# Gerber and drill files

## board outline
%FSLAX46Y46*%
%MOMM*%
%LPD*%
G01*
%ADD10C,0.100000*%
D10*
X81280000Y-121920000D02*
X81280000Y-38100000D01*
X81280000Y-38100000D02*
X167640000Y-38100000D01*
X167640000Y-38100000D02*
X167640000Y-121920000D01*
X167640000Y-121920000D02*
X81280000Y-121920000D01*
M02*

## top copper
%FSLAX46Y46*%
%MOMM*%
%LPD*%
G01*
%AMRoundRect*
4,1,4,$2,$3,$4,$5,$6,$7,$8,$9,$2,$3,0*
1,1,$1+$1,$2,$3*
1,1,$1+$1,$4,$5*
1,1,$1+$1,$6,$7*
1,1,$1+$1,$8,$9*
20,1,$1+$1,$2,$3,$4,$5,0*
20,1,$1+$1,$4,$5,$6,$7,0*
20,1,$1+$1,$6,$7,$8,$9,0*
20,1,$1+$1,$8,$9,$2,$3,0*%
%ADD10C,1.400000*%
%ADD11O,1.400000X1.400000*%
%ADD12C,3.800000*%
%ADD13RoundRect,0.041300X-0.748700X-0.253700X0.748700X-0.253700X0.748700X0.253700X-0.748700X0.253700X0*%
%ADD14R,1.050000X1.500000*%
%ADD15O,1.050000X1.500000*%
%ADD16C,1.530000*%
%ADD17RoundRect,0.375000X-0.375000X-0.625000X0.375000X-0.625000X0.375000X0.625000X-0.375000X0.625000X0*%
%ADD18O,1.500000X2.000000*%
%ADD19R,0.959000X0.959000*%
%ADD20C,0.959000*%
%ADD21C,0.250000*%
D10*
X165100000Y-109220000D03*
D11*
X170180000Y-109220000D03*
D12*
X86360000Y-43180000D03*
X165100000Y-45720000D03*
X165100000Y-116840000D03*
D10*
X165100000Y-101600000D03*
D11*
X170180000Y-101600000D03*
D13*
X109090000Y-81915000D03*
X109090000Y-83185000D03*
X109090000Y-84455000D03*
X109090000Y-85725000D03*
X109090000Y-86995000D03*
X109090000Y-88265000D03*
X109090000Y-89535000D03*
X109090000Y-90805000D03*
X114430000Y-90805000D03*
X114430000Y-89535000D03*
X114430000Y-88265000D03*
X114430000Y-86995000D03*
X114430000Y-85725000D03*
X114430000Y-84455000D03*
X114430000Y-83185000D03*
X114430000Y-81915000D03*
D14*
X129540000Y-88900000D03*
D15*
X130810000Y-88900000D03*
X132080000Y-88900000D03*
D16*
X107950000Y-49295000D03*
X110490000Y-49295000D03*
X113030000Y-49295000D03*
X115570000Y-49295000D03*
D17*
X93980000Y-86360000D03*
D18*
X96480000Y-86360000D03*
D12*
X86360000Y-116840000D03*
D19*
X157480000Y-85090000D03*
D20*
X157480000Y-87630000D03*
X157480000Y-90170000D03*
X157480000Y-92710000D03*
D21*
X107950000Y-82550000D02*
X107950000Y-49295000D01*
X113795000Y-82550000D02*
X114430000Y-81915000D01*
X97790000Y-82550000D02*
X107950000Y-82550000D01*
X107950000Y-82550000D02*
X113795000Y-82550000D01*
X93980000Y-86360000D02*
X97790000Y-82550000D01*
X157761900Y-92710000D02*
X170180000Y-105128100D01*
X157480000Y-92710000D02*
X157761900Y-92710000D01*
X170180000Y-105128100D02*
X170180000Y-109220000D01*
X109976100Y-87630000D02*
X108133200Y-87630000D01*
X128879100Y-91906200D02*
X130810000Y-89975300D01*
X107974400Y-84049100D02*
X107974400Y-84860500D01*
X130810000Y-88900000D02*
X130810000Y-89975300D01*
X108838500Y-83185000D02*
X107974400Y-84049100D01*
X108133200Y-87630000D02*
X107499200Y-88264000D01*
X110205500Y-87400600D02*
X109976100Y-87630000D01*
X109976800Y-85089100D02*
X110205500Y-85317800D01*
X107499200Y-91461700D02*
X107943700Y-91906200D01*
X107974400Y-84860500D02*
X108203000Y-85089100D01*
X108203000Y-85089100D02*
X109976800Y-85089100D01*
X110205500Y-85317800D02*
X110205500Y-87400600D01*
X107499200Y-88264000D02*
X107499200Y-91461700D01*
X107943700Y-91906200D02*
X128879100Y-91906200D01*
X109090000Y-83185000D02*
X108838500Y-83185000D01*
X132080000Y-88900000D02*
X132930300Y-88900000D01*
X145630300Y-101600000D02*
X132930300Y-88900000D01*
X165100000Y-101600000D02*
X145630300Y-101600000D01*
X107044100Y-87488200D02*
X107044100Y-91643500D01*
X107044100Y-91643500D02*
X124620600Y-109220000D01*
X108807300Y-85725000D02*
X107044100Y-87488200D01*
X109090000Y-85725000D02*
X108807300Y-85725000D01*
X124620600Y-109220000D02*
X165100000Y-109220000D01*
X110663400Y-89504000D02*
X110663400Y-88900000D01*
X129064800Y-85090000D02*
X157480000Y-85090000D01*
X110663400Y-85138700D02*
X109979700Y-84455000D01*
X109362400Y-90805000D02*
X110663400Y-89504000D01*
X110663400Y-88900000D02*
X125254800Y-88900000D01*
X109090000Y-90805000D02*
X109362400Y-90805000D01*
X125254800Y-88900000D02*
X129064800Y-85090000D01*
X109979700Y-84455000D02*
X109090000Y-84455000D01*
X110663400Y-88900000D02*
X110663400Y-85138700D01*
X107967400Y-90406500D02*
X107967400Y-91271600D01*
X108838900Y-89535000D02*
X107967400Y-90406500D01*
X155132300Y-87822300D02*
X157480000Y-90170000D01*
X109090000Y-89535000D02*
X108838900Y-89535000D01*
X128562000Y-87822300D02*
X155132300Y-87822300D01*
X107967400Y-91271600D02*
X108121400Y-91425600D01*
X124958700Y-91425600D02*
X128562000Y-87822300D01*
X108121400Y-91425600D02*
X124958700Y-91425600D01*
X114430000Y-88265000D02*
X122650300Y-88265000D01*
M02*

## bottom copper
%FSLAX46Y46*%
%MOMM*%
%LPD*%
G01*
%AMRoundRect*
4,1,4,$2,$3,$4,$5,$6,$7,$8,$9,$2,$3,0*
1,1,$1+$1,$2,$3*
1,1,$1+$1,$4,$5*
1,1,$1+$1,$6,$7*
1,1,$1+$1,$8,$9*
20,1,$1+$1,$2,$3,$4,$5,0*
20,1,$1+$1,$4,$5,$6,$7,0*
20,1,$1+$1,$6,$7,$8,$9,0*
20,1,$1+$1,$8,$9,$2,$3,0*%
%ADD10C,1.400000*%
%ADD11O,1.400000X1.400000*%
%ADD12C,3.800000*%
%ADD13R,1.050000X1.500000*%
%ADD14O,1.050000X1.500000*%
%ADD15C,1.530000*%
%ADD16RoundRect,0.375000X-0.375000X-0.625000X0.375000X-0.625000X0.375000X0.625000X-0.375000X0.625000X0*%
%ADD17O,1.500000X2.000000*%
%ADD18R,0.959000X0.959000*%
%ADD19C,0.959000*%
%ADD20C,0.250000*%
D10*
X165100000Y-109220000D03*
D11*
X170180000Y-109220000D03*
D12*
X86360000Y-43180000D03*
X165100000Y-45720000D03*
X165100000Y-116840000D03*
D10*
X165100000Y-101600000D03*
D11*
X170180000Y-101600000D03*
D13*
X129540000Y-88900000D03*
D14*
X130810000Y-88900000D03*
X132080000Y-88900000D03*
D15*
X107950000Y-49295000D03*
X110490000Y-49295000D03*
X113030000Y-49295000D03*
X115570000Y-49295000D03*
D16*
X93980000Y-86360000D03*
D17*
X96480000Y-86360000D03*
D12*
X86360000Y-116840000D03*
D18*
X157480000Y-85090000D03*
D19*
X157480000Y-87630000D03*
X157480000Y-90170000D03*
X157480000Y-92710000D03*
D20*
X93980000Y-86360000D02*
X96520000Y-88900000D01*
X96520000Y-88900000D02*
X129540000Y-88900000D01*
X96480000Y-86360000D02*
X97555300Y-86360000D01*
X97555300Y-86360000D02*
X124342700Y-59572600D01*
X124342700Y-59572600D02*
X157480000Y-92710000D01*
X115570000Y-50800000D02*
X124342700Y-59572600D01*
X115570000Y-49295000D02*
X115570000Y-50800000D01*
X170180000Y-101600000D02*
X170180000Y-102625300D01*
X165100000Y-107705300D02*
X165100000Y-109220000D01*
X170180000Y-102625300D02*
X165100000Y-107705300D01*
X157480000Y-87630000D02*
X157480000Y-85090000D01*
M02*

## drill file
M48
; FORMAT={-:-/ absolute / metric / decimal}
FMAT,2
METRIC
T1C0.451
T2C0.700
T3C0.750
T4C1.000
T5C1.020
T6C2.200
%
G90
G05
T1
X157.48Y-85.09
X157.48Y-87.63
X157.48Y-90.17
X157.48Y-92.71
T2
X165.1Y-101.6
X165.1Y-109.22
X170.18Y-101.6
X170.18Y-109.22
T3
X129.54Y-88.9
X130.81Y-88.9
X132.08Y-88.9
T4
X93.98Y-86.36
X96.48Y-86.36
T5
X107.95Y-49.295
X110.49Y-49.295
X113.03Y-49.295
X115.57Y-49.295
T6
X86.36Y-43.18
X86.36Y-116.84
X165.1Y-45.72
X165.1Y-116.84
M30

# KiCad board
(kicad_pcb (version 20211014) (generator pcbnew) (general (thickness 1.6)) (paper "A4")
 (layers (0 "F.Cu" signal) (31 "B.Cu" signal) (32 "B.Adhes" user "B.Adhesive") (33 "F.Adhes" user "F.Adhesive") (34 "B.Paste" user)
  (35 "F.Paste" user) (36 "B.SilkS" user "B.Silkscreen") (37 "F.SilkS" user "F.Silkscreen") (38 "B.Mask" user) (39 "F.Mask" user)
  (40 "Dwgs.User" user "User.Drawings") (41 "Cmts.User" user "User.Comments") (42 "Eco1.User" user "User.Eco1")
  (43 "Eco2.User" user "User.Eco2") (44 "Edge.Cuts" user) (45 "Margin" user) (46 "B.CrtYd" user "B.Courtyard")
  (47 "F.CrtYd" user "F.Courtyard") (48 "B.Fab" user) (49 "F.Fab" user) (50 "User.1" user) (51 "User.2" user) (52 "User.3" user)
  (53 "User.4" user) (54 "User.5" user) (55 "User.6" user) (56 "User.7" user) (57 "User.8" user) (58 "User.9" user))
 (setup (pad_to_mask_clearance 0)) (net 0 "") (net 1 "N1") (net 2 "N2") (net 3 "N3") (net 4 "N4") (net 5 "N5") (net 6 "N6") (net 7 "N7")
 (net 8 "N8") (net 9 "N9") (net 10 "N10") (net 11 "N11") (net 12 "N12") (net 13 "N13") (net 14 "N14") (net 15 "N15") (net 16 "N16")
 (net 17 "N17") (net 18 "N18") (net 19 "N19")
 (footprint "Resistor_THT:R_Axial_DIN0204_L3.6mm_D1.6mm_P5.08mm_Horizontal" (layer "F.Cu") (at 165.1 109.22)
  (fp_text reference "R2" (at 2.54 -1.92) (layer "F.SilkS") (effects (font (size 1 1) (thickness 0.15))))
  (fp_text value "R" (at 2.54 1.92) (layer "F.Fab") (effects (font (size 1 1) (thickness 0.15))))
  (pad "1" thru_hole circle (at 0 0) (size 1.4 1.4) (drill 0.7) (layers *.Cu *.Mask) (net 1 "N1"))
  (pad "2" thru_hole oval (at 5.08 0) (size 1.4 1.4) (drill 0.7) (layers *.Cu *.Mask) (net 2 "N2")))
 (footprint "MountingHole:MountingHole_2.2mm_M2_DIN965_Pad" (layer "F.Cu") (at 86.36 43.18)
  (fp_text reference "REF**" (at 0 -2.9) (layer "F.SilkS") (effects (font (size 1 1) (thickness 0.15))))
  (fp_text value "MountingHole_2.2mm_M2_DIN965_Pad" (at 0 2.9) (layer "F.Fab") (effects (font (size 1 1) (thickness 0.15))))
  (pad "1" thru_hole circle (at 0 0) (size 3.8 3.8) (drill 2.2) (layers *.Cu *.Mask)))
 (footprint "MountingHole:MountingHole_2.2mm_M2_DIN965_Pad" (layer "F.Cu") (at 165.1 45.72)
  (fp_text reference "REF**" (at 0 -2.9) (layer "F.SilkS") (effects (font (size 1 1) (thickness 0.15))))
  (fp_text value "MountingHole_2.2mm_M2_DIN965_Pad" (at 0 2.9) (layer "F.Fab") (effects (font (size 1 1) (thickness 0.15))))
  (pad "1" thru_hole circle (at 0 0) (size 3.8 3.8) (drill 2.2) (layers *.Cu *.Mask)))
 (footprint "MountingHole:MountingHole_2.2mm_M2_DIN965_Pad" (layer "F.Cu") (at 165.1 116.84)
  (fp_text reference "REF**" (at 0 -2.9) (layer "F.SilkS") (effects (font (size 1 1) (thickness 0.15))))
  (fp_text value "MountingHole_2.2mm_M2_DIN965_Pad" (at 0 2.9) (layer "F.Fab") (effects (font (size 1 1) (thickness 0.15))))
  (pad "1" thru_hole circle (at 0 0) (size 3.8 3.8) (drill 2.2) (layers *.Cu *.Mask)))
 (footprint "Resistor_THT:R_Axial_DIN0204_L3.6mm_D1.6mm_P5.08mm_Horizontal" (layer "F.Cu") (at 165.1 101.6)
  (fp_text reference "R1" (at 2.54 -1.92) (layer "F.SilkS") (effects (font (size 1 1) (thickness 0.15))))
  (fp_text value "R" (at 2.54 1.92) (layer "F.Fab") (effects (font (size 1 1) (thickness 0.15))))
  (pad "1" thru_hole circle (at 0 0) (size 1.4 1.4) (drill 0.7) (layers *.Cu *.Mask) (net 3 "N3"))
  (pad "2" thru_hole oval (at 5.08 0) (size 1.4 1.4) (drill 0.7) (layers *.Cu *.Mask) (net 1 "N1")))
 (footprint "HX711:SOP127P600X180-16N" (layer "F.Cu") (at 111.76 86.36)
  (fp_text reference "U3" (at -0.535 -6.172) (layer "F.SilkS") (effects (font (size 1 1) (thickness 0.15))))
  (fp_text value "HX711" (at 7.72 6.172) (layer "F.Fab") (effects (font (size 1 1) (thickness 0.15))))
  (pad "1" smd roundrect locked (at -2.67 -4.445) (size 1.58 0.59) (layers "F.Cu" "F.Paste" "F.Mask") (roundrect_rratio 0.07) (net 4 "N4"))
  (pad "2" smd roundrect locked (at -2.67 -3.175) (size 1.58 0.59) (layers "F.Cu" "F.Paste" "F.Mask") (roundrect_rratio 0.07) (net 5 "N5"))
  (pad "3" smd roundrect locked (at -2.67 -1.905) (size 1.58 0.59) (layers "F.Cu" "F.Paste" "F.Mask") (roundrect_rratio 0.07) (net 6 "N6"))
  (pad "4" smd roundrect locked (at -2.67 -0.635) (size 1.58 0.59) (layers "F.Cu" "F.Paste" "F.Mask") (roundrect_rratio 0.07) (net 1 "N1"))
  (pad "5" smd roundrect locked (at -2.67 0.635) (size 1.58 0.59) (layers "F.Cu" "F.Paste" "F.Mask") (roundrect_rratio 0.07) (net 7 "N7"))
  (pad "6" smd roundrect locked (at -2.67 1.905) (size 1.58 0.59) (layers "F.Cu" "F.Paste" "F.Mask") (roundrect_rratio 0.07) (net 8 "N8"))
  (pad "7" smd roundrect locked (at -2.67 3.175) (size 1.58 0.59) (layers "F.Cu" "F.Paste" "F.Mask") (roundrect_rratio 0.07) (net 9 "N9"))
  (pad "8" smd roundrect locked (at -2.67 4.445) (size 1.58 0.59) (layers "F.Cu" "F.Paste" "F.Mask") (roundrect_rratio 0.07) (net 6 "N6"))
  (pad "9" smd roundrect locked (at 2.67 4.445) (size 1.58 0.59) (layers "F.Cu" "F.Paste" "F.Mask") (roundrect_rratio 0.07) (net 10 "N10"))
  (pad "10" smd roundrect locked (at 2.67 3.175) (size 1.58 0.59) (layers "F.Cu" "F.Paste" "F.Mask") (roundrect_rratio 0.07) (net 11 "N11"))
  (pad "11" smd roundrect locked (at 2.67 1.905) (size 1.58 0.59) (layers "F.Cu" "F.Paste" "F.Mask") (roundrect_rratio 0.07) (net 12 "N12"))
  (pad "12" smd roundrect locked (at 2.67 0.635) (size 1.58 0.59) (layers "F.Cu" "F.Paste" "F.Mask") (roundrect_rratio 0.07) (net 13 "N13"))
  (pad "13" smd roundrect locked (at 2.67 -0.635) (size 1.58 0.59) (layers "F.Cu" "F.Paste" "F.Mask") (roundrect_rratio 0.07) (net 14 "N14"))
  (pad "14" smd roundrect locked (at 2.67 -1.905) (size 1.58 0.59) (layers "F.Cu" "F.Paste" "F.Mask") (roundrect_rratio 0.07) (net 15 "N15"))
  (pad "15" smd roundrect locked (at 2.67 -3.175) (size 1.58 0.59) (layers "F.Cu" "F.Paste" "F.Mask") (roundrect_rratio 0.07) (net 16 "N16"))
  (pad "16" smd roundrect locked (at 2.67 -4.445) (size 1.58 0.59) (layers "F.Cu" "F.Paste" "F.Mask") (roundrect_rratio 0.07) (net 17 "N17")))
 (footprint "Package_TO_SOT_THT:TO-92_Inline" (layer "F.Cu") (at 129.54 88.9)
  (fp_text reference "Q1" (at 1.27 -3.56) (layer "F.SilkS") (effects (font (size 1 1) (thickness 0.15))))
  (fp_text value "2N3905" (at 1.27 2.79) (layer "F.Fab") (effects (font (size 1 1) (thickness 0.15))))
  (pad "1" thru_hole rect (at 0 0) (size 1.05 1.5) (drill 0.75) (layers *.Cu *.Mask) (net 17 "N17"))
  (pad "2" thru_hole oval (at 1.27 0) (size 1.05 1.5) (drill 0.75) (layers *.Cu *.Mask) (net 5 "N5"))
  (pad "3" thru_hole oval (at 2.54 0) (size 1.05 1.5) (drill 0.75) (layers *.Cu *.Mask) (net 3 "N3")))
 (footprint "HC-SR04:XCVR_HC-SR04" (layer "F.Cu") (at 111.76 49.295)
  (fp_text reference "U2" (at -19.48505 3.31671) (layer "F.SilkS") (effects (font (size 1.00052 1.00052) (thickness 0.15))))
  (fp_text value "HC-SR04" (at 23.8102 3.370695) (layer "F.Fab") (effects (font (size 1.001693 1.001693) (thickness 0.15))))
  (pad "1" thru_hole circle locked (at -3.81 0) (size 1.53 1.53) (drill 1.02) (layers *.Cu *.Mask) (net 17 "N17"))
  (pad "2" thru_hole circle locked (at -1.27 0) (size 1.53 1.53) (drill 1.02) (layers *.Cu *.Mask) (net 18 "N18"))
  (pad "3" thru_hole circle locked (at 1.27 0) (size 1.53 1.53) (drill 1.02) (layers *.Cu *.Mask) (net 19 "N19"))
  (pad "4" thru_hole circle locked (at 3.81 0) (size 1.53 1.53) (drill 1.02) (layers *.Cu *.Mask) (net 2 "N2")))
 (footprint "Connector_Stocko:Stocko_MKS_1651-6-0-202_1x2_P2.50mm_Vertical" (layer "F.Cu") (at 93.98 86.36)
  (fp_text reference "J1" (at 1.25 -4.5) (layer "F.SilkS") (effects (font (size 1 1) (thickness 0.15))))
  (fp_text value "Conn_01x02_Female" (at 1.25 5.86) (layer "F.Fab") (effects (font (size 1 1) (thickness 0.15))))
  (pad "1" thru_hole roundrect (at 0 0) (size 1.5 2) (drill 1) (layers *.Cu *.Mask) (roundrect_rratio 0.25) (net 17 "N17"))
  (pad "2" thru_hole oval (at 2.5 0) (size 1.5 2) (drill 1) (layers *.Cu *.Mask) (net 2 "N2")))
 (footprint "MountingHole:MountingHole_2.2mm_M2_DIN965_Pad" (layer "F.Cu") (at 86.36 116.84)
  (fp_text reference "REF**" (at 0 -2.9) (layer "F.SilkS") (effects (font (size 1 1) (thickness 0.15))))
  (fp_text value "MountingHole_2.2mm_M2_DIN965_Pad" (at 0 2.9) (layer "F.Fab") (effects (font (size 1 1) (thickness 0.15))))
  (pad "1" thru_hole circle (at 0 0) (size 3.8 3.8) (drill 2.2) (layers *.Cu *.Mask)))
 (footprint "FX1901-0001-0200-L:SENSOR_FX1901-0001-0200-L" (layer "F.Cu") (at 157.48 88.9)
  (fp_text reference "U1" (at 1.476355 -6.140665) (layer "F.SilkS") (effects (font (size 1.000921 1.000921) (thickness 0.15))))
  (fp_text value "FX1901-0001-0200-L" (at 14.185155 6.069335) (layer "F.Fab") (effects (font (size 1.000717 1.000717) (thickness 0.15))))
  (pad "1" thru_hole rect locked (at 0 -3.81) (size 0.959 0.959) (drill 0.451) (layers *.Cu *.Mask) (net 6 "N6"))
  (pad "2" thru_hole circle locked (at 0 -1.27) (size 0.959 0.959) (drill 0.451) (layers *.Cu *.Mask) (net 6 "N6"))
  (pad "3" thru_hole circle locked (at 0 1.27) (size 0.959 0.959) (drill 0.451) (layers *.Cu *.Mask) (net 9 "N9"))
  (pad "4" thru_hole circle locked (at 0 3.81) (size 0.959 0.959) (drill 0.451) (layers *.Cu *.Mask) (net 2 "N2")))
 (gr_line (start 81.28 121.92) (end 81.28 38.1) (layer "Edge.Cuts") (width 0.1))
 (gr_line (start 81.28 38.1) (end 167.64 38.1) (layer "Edge.Cuts") (width 0.1))
 (gr_line (start 167.64 38.1) (end 167.64 121.92) (layer "Edge.Cuts") (width 0.1))
 (gr_line (start 167.64 121.92) (end 81.28 121.92) (layer "Edge.Cuts") (width 0.1))
 (segment (start 107.95 82.55) (end 107.95 49.295) (width 0.25) (layer "F.Cu") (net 17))
 (segment (start 113.795 82.55) (end 114.43 81.915) (width 0.25) (layer "F.Cu") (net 17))
 (segment (start 97.79 82.55) (end 107.95 82.55) (width 0.25) (layer "F.Cu") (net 17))
 (segment (start 107.95 82.55) (end 113.795 82.55) (width 0.25) (layer "F.Cu") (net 17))
 (segment (start 93.98 86.36) (end 97.79 82.55) (width 0.25) (layer "F.Cu") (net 17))
 (segment (start 93.98 86.36) (end 96.52 88.9) (width 0.25) (layer "B.Cu") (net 17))
 (segment (start 96.52 88.9) (end 129.54 88.9) (width 0.25) (layer "B.Cu") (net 17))
 (segment (start 157.7619 92.71) (end 170.18 105.1281) (width 0.25) (layer "F.Cu") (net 2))
 (segment (start 157.48 92.71) (end 157.7619 92.71) (width 0.25) (layer "F.Cu") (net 2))
 (segment (start 170.18 105.1281) (end 170.18 109.22) (width 0.25) (layer "F.Cu") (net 2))
 (segment (start 96.48 86.36) (end 97.5553 86.36) (width 0.25) (layer "B.Cu") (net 2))
 (segment (start 97.5553 86.36) (end 124.3427 59.5726) (width 0.25) (layer "B.Cu") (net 2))
 (segment (start 124.3427 59.5726) (end 157.48 92.71) (width 0.25) (layer "B.Cu") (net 2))
 (segment (start 115.57 50.8) (end 124.3427 59.5726) (width 0.25) (layer "B.Cu") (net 2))
 (segment (start 115.57 49.295) (end 115.57 50.8) (width 0.25) (layer "B.Cu") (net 2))
 (segment (start 109.9761 87.63) (end 108.1332 87.63) (width 0.25) (layer "F.Cu") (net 5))
 (segment (start 128.8791 91.9062) (end 130.81 89.9753) (width 0.25) (layer "F.Cu") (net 5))
 (segment (start 107.9744 84.0491) (end 107.9744 84.8605) (width 0.25) (layer "F.Cu") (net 5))
 (segment (start 130.81 88.9) (end 130.81 89.9753) (width 0.25) (layer "F.Cu") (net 5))
 (segment (start 108.8385 83.185) (end 107.9744 84.0491) (width 0.25) (layer "F.Cu") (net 5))
 (segment (start 108.1332 87.63) (end 107.4992 88.264) (width 0.25) (layer "F.Cu") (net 5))
 (segment (start 110.2055 87.4006) (end 109.9761 87.63) (width 0.25) (layer "F.Cu") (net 5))
 (segment (start 109.9768 85.0891) (end 110.2055 85.3178) (width 0.25) (layer "F.Cu") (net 5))
 (segment (start 107.4992 91.4617) (end 107.9437 91.9062) (width 0.25) (layer "F.Cu") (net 5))
 (segment (start 107.9744 84.8605) (end 108.203 85.0891) (width 0.25) (layer "F.Cu") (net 5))
 (segment (start 108.203 85.0891) (end 109.9768 85.0891) (width 0.25) (layer "F.Cu") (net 5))
 (segment (start 110.2055 85.3178) (end 110.2055 87.4006) (width 0.25) (layer "F.Cu") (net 5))
 (segment (start 107.4992 88.264) (end 107.4992 91.4617) (width 0.25) (layer "F.Cu") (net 5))
 (segment (start 107.9437 91.9062) (end 128.8791 91.9062) (width 0.25) (layer "F.Cu") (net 5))
 (segment (start 109.09 83.185) (end 108.8385 83.185) (width 0.25) (layer "F.Cu") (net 5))
 (segment (start 132.08 88.9) (end 132.9303 88.9) (width 0.25) (layer "F.Cu") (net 3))
 (segment (start 145.6303 101.6) (end 132.9303 88.9) (width 0.25) (layer "F.Cu") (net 3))
 (segment (start 165.1 101.6) (end 145.6303 101.6) (width 0.25) (layer "F.Cu") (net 3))
 (segment (start 107.0441 87.4882) (end 107.0441 91.6435) (width 0.25) (layer "F.Cu") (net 1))
 (segment (start 107.0441 91.6435) (end 124.6206 109.22) (width 0.25) (layer "F.Cu") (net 1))
 (segment (start 108.8073 85.725) (end 107.0441 87.4882) (width 0.25) (layer "F.Cu") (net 1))
 (segment (start 109.09 85.725) (end 108.8073 85.725) (width 0.25) (layer "F.Cu") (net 1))
 (segment (start 124.6206 109.22) (end 165.1 109.22) (width 0.25) (layer "F.Cu") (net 1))
 (segment (start 170.18 101.6) (end 170.18 102.6253) (width 0.25) (layer "B.Cu") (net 1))
 (segment (start 165.1 107.7053) (end 165.1 109.22) (width 0.25) (layer "B.Cu") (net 1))
 (segment (start 170.18 102.6253) (end 165.1 107.7053) (width 0.25) (layer "B.Cu") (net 1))
 (segment (start 110.6634 89.504) (end 110.6634 88.9) (width 0.25) (layer "F.Cu") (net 6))
 (segment (start 129.0648 85.09) (end 157.48 85.09) (width 0.25) (layer "F.Cu") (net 6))
 (segment (start 110.6634 85.1387) (end 109.9797 84.455) (width 0.25) (layer "F.Cu") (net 6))
 (segment (start 109.3624 90.805) (end 110.6634 89.504) (width 0.25) (layer "F.Cu") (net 6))
 (segment (start 110.6634 88.9) (end 125.2548 88.9) (width 0.25) (layer "F.Cu") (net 6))
 (segment (start 109.09 90.805) (end 109.3624 90.805) (width 0.25) (layer "F.Cu") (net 6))
 (segment (start 125.2548 88.9) (end 129.0648 85.09) (width 0.25) (layer "F.Cu") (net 6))
 (segment (start 109.9797 84.455) (end 109.09 84.455) (width 0.25) (layer "F.Cu") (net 6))
 (segment (start 110.6634 88.9) (end 110.6634 85.1387) (width 0.25) (layer "F.Cu") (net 6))
 (segment (start 157.48 87.63) (end 157.48 85.09) (width 0.25) (layer "B.Cu") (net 6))
 (segment (start 107.9674 90.4065) (end 107.9674 91.2716) (width 0.25) (layer "F.Cu") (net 9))
 (segment (start 108.8389 89.535) (end 107.9674 90.4065) (width 0.25) (layer "F.Cu") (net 9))
 (segment (start 155.1323 87.8223) (end 157.48 90.17) (width 0.25) (layer "F.Cu") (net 9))
 (segment (start 109.09 89.535) (end 108.8389 89.535) (width 0.25) (layer "F.Cu") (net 9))
 (segment (start 128.562 87.8223) (end 155.1323 87.8223) (width 0.25) (layer "F.Cu") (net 9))
 (segment (start 107.9674 91.2716) (end 108.1214 91.4256) (width 0.25) (layer "F.Cu") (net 9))
 (segment (start 124.9587 91.4256) (end 128.562 87.8223) (width 0.25) (layer "F.Cu") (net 9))
 (segment (start 108.1214 91.4256) (end 124.9587 91.4256) (width 0.25) (layer "F.Cu") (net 9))
 (segment (start 114.43 88.265) (end 122.6503 88.265) (width 0.25) (layer "F.Cu") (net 12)))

